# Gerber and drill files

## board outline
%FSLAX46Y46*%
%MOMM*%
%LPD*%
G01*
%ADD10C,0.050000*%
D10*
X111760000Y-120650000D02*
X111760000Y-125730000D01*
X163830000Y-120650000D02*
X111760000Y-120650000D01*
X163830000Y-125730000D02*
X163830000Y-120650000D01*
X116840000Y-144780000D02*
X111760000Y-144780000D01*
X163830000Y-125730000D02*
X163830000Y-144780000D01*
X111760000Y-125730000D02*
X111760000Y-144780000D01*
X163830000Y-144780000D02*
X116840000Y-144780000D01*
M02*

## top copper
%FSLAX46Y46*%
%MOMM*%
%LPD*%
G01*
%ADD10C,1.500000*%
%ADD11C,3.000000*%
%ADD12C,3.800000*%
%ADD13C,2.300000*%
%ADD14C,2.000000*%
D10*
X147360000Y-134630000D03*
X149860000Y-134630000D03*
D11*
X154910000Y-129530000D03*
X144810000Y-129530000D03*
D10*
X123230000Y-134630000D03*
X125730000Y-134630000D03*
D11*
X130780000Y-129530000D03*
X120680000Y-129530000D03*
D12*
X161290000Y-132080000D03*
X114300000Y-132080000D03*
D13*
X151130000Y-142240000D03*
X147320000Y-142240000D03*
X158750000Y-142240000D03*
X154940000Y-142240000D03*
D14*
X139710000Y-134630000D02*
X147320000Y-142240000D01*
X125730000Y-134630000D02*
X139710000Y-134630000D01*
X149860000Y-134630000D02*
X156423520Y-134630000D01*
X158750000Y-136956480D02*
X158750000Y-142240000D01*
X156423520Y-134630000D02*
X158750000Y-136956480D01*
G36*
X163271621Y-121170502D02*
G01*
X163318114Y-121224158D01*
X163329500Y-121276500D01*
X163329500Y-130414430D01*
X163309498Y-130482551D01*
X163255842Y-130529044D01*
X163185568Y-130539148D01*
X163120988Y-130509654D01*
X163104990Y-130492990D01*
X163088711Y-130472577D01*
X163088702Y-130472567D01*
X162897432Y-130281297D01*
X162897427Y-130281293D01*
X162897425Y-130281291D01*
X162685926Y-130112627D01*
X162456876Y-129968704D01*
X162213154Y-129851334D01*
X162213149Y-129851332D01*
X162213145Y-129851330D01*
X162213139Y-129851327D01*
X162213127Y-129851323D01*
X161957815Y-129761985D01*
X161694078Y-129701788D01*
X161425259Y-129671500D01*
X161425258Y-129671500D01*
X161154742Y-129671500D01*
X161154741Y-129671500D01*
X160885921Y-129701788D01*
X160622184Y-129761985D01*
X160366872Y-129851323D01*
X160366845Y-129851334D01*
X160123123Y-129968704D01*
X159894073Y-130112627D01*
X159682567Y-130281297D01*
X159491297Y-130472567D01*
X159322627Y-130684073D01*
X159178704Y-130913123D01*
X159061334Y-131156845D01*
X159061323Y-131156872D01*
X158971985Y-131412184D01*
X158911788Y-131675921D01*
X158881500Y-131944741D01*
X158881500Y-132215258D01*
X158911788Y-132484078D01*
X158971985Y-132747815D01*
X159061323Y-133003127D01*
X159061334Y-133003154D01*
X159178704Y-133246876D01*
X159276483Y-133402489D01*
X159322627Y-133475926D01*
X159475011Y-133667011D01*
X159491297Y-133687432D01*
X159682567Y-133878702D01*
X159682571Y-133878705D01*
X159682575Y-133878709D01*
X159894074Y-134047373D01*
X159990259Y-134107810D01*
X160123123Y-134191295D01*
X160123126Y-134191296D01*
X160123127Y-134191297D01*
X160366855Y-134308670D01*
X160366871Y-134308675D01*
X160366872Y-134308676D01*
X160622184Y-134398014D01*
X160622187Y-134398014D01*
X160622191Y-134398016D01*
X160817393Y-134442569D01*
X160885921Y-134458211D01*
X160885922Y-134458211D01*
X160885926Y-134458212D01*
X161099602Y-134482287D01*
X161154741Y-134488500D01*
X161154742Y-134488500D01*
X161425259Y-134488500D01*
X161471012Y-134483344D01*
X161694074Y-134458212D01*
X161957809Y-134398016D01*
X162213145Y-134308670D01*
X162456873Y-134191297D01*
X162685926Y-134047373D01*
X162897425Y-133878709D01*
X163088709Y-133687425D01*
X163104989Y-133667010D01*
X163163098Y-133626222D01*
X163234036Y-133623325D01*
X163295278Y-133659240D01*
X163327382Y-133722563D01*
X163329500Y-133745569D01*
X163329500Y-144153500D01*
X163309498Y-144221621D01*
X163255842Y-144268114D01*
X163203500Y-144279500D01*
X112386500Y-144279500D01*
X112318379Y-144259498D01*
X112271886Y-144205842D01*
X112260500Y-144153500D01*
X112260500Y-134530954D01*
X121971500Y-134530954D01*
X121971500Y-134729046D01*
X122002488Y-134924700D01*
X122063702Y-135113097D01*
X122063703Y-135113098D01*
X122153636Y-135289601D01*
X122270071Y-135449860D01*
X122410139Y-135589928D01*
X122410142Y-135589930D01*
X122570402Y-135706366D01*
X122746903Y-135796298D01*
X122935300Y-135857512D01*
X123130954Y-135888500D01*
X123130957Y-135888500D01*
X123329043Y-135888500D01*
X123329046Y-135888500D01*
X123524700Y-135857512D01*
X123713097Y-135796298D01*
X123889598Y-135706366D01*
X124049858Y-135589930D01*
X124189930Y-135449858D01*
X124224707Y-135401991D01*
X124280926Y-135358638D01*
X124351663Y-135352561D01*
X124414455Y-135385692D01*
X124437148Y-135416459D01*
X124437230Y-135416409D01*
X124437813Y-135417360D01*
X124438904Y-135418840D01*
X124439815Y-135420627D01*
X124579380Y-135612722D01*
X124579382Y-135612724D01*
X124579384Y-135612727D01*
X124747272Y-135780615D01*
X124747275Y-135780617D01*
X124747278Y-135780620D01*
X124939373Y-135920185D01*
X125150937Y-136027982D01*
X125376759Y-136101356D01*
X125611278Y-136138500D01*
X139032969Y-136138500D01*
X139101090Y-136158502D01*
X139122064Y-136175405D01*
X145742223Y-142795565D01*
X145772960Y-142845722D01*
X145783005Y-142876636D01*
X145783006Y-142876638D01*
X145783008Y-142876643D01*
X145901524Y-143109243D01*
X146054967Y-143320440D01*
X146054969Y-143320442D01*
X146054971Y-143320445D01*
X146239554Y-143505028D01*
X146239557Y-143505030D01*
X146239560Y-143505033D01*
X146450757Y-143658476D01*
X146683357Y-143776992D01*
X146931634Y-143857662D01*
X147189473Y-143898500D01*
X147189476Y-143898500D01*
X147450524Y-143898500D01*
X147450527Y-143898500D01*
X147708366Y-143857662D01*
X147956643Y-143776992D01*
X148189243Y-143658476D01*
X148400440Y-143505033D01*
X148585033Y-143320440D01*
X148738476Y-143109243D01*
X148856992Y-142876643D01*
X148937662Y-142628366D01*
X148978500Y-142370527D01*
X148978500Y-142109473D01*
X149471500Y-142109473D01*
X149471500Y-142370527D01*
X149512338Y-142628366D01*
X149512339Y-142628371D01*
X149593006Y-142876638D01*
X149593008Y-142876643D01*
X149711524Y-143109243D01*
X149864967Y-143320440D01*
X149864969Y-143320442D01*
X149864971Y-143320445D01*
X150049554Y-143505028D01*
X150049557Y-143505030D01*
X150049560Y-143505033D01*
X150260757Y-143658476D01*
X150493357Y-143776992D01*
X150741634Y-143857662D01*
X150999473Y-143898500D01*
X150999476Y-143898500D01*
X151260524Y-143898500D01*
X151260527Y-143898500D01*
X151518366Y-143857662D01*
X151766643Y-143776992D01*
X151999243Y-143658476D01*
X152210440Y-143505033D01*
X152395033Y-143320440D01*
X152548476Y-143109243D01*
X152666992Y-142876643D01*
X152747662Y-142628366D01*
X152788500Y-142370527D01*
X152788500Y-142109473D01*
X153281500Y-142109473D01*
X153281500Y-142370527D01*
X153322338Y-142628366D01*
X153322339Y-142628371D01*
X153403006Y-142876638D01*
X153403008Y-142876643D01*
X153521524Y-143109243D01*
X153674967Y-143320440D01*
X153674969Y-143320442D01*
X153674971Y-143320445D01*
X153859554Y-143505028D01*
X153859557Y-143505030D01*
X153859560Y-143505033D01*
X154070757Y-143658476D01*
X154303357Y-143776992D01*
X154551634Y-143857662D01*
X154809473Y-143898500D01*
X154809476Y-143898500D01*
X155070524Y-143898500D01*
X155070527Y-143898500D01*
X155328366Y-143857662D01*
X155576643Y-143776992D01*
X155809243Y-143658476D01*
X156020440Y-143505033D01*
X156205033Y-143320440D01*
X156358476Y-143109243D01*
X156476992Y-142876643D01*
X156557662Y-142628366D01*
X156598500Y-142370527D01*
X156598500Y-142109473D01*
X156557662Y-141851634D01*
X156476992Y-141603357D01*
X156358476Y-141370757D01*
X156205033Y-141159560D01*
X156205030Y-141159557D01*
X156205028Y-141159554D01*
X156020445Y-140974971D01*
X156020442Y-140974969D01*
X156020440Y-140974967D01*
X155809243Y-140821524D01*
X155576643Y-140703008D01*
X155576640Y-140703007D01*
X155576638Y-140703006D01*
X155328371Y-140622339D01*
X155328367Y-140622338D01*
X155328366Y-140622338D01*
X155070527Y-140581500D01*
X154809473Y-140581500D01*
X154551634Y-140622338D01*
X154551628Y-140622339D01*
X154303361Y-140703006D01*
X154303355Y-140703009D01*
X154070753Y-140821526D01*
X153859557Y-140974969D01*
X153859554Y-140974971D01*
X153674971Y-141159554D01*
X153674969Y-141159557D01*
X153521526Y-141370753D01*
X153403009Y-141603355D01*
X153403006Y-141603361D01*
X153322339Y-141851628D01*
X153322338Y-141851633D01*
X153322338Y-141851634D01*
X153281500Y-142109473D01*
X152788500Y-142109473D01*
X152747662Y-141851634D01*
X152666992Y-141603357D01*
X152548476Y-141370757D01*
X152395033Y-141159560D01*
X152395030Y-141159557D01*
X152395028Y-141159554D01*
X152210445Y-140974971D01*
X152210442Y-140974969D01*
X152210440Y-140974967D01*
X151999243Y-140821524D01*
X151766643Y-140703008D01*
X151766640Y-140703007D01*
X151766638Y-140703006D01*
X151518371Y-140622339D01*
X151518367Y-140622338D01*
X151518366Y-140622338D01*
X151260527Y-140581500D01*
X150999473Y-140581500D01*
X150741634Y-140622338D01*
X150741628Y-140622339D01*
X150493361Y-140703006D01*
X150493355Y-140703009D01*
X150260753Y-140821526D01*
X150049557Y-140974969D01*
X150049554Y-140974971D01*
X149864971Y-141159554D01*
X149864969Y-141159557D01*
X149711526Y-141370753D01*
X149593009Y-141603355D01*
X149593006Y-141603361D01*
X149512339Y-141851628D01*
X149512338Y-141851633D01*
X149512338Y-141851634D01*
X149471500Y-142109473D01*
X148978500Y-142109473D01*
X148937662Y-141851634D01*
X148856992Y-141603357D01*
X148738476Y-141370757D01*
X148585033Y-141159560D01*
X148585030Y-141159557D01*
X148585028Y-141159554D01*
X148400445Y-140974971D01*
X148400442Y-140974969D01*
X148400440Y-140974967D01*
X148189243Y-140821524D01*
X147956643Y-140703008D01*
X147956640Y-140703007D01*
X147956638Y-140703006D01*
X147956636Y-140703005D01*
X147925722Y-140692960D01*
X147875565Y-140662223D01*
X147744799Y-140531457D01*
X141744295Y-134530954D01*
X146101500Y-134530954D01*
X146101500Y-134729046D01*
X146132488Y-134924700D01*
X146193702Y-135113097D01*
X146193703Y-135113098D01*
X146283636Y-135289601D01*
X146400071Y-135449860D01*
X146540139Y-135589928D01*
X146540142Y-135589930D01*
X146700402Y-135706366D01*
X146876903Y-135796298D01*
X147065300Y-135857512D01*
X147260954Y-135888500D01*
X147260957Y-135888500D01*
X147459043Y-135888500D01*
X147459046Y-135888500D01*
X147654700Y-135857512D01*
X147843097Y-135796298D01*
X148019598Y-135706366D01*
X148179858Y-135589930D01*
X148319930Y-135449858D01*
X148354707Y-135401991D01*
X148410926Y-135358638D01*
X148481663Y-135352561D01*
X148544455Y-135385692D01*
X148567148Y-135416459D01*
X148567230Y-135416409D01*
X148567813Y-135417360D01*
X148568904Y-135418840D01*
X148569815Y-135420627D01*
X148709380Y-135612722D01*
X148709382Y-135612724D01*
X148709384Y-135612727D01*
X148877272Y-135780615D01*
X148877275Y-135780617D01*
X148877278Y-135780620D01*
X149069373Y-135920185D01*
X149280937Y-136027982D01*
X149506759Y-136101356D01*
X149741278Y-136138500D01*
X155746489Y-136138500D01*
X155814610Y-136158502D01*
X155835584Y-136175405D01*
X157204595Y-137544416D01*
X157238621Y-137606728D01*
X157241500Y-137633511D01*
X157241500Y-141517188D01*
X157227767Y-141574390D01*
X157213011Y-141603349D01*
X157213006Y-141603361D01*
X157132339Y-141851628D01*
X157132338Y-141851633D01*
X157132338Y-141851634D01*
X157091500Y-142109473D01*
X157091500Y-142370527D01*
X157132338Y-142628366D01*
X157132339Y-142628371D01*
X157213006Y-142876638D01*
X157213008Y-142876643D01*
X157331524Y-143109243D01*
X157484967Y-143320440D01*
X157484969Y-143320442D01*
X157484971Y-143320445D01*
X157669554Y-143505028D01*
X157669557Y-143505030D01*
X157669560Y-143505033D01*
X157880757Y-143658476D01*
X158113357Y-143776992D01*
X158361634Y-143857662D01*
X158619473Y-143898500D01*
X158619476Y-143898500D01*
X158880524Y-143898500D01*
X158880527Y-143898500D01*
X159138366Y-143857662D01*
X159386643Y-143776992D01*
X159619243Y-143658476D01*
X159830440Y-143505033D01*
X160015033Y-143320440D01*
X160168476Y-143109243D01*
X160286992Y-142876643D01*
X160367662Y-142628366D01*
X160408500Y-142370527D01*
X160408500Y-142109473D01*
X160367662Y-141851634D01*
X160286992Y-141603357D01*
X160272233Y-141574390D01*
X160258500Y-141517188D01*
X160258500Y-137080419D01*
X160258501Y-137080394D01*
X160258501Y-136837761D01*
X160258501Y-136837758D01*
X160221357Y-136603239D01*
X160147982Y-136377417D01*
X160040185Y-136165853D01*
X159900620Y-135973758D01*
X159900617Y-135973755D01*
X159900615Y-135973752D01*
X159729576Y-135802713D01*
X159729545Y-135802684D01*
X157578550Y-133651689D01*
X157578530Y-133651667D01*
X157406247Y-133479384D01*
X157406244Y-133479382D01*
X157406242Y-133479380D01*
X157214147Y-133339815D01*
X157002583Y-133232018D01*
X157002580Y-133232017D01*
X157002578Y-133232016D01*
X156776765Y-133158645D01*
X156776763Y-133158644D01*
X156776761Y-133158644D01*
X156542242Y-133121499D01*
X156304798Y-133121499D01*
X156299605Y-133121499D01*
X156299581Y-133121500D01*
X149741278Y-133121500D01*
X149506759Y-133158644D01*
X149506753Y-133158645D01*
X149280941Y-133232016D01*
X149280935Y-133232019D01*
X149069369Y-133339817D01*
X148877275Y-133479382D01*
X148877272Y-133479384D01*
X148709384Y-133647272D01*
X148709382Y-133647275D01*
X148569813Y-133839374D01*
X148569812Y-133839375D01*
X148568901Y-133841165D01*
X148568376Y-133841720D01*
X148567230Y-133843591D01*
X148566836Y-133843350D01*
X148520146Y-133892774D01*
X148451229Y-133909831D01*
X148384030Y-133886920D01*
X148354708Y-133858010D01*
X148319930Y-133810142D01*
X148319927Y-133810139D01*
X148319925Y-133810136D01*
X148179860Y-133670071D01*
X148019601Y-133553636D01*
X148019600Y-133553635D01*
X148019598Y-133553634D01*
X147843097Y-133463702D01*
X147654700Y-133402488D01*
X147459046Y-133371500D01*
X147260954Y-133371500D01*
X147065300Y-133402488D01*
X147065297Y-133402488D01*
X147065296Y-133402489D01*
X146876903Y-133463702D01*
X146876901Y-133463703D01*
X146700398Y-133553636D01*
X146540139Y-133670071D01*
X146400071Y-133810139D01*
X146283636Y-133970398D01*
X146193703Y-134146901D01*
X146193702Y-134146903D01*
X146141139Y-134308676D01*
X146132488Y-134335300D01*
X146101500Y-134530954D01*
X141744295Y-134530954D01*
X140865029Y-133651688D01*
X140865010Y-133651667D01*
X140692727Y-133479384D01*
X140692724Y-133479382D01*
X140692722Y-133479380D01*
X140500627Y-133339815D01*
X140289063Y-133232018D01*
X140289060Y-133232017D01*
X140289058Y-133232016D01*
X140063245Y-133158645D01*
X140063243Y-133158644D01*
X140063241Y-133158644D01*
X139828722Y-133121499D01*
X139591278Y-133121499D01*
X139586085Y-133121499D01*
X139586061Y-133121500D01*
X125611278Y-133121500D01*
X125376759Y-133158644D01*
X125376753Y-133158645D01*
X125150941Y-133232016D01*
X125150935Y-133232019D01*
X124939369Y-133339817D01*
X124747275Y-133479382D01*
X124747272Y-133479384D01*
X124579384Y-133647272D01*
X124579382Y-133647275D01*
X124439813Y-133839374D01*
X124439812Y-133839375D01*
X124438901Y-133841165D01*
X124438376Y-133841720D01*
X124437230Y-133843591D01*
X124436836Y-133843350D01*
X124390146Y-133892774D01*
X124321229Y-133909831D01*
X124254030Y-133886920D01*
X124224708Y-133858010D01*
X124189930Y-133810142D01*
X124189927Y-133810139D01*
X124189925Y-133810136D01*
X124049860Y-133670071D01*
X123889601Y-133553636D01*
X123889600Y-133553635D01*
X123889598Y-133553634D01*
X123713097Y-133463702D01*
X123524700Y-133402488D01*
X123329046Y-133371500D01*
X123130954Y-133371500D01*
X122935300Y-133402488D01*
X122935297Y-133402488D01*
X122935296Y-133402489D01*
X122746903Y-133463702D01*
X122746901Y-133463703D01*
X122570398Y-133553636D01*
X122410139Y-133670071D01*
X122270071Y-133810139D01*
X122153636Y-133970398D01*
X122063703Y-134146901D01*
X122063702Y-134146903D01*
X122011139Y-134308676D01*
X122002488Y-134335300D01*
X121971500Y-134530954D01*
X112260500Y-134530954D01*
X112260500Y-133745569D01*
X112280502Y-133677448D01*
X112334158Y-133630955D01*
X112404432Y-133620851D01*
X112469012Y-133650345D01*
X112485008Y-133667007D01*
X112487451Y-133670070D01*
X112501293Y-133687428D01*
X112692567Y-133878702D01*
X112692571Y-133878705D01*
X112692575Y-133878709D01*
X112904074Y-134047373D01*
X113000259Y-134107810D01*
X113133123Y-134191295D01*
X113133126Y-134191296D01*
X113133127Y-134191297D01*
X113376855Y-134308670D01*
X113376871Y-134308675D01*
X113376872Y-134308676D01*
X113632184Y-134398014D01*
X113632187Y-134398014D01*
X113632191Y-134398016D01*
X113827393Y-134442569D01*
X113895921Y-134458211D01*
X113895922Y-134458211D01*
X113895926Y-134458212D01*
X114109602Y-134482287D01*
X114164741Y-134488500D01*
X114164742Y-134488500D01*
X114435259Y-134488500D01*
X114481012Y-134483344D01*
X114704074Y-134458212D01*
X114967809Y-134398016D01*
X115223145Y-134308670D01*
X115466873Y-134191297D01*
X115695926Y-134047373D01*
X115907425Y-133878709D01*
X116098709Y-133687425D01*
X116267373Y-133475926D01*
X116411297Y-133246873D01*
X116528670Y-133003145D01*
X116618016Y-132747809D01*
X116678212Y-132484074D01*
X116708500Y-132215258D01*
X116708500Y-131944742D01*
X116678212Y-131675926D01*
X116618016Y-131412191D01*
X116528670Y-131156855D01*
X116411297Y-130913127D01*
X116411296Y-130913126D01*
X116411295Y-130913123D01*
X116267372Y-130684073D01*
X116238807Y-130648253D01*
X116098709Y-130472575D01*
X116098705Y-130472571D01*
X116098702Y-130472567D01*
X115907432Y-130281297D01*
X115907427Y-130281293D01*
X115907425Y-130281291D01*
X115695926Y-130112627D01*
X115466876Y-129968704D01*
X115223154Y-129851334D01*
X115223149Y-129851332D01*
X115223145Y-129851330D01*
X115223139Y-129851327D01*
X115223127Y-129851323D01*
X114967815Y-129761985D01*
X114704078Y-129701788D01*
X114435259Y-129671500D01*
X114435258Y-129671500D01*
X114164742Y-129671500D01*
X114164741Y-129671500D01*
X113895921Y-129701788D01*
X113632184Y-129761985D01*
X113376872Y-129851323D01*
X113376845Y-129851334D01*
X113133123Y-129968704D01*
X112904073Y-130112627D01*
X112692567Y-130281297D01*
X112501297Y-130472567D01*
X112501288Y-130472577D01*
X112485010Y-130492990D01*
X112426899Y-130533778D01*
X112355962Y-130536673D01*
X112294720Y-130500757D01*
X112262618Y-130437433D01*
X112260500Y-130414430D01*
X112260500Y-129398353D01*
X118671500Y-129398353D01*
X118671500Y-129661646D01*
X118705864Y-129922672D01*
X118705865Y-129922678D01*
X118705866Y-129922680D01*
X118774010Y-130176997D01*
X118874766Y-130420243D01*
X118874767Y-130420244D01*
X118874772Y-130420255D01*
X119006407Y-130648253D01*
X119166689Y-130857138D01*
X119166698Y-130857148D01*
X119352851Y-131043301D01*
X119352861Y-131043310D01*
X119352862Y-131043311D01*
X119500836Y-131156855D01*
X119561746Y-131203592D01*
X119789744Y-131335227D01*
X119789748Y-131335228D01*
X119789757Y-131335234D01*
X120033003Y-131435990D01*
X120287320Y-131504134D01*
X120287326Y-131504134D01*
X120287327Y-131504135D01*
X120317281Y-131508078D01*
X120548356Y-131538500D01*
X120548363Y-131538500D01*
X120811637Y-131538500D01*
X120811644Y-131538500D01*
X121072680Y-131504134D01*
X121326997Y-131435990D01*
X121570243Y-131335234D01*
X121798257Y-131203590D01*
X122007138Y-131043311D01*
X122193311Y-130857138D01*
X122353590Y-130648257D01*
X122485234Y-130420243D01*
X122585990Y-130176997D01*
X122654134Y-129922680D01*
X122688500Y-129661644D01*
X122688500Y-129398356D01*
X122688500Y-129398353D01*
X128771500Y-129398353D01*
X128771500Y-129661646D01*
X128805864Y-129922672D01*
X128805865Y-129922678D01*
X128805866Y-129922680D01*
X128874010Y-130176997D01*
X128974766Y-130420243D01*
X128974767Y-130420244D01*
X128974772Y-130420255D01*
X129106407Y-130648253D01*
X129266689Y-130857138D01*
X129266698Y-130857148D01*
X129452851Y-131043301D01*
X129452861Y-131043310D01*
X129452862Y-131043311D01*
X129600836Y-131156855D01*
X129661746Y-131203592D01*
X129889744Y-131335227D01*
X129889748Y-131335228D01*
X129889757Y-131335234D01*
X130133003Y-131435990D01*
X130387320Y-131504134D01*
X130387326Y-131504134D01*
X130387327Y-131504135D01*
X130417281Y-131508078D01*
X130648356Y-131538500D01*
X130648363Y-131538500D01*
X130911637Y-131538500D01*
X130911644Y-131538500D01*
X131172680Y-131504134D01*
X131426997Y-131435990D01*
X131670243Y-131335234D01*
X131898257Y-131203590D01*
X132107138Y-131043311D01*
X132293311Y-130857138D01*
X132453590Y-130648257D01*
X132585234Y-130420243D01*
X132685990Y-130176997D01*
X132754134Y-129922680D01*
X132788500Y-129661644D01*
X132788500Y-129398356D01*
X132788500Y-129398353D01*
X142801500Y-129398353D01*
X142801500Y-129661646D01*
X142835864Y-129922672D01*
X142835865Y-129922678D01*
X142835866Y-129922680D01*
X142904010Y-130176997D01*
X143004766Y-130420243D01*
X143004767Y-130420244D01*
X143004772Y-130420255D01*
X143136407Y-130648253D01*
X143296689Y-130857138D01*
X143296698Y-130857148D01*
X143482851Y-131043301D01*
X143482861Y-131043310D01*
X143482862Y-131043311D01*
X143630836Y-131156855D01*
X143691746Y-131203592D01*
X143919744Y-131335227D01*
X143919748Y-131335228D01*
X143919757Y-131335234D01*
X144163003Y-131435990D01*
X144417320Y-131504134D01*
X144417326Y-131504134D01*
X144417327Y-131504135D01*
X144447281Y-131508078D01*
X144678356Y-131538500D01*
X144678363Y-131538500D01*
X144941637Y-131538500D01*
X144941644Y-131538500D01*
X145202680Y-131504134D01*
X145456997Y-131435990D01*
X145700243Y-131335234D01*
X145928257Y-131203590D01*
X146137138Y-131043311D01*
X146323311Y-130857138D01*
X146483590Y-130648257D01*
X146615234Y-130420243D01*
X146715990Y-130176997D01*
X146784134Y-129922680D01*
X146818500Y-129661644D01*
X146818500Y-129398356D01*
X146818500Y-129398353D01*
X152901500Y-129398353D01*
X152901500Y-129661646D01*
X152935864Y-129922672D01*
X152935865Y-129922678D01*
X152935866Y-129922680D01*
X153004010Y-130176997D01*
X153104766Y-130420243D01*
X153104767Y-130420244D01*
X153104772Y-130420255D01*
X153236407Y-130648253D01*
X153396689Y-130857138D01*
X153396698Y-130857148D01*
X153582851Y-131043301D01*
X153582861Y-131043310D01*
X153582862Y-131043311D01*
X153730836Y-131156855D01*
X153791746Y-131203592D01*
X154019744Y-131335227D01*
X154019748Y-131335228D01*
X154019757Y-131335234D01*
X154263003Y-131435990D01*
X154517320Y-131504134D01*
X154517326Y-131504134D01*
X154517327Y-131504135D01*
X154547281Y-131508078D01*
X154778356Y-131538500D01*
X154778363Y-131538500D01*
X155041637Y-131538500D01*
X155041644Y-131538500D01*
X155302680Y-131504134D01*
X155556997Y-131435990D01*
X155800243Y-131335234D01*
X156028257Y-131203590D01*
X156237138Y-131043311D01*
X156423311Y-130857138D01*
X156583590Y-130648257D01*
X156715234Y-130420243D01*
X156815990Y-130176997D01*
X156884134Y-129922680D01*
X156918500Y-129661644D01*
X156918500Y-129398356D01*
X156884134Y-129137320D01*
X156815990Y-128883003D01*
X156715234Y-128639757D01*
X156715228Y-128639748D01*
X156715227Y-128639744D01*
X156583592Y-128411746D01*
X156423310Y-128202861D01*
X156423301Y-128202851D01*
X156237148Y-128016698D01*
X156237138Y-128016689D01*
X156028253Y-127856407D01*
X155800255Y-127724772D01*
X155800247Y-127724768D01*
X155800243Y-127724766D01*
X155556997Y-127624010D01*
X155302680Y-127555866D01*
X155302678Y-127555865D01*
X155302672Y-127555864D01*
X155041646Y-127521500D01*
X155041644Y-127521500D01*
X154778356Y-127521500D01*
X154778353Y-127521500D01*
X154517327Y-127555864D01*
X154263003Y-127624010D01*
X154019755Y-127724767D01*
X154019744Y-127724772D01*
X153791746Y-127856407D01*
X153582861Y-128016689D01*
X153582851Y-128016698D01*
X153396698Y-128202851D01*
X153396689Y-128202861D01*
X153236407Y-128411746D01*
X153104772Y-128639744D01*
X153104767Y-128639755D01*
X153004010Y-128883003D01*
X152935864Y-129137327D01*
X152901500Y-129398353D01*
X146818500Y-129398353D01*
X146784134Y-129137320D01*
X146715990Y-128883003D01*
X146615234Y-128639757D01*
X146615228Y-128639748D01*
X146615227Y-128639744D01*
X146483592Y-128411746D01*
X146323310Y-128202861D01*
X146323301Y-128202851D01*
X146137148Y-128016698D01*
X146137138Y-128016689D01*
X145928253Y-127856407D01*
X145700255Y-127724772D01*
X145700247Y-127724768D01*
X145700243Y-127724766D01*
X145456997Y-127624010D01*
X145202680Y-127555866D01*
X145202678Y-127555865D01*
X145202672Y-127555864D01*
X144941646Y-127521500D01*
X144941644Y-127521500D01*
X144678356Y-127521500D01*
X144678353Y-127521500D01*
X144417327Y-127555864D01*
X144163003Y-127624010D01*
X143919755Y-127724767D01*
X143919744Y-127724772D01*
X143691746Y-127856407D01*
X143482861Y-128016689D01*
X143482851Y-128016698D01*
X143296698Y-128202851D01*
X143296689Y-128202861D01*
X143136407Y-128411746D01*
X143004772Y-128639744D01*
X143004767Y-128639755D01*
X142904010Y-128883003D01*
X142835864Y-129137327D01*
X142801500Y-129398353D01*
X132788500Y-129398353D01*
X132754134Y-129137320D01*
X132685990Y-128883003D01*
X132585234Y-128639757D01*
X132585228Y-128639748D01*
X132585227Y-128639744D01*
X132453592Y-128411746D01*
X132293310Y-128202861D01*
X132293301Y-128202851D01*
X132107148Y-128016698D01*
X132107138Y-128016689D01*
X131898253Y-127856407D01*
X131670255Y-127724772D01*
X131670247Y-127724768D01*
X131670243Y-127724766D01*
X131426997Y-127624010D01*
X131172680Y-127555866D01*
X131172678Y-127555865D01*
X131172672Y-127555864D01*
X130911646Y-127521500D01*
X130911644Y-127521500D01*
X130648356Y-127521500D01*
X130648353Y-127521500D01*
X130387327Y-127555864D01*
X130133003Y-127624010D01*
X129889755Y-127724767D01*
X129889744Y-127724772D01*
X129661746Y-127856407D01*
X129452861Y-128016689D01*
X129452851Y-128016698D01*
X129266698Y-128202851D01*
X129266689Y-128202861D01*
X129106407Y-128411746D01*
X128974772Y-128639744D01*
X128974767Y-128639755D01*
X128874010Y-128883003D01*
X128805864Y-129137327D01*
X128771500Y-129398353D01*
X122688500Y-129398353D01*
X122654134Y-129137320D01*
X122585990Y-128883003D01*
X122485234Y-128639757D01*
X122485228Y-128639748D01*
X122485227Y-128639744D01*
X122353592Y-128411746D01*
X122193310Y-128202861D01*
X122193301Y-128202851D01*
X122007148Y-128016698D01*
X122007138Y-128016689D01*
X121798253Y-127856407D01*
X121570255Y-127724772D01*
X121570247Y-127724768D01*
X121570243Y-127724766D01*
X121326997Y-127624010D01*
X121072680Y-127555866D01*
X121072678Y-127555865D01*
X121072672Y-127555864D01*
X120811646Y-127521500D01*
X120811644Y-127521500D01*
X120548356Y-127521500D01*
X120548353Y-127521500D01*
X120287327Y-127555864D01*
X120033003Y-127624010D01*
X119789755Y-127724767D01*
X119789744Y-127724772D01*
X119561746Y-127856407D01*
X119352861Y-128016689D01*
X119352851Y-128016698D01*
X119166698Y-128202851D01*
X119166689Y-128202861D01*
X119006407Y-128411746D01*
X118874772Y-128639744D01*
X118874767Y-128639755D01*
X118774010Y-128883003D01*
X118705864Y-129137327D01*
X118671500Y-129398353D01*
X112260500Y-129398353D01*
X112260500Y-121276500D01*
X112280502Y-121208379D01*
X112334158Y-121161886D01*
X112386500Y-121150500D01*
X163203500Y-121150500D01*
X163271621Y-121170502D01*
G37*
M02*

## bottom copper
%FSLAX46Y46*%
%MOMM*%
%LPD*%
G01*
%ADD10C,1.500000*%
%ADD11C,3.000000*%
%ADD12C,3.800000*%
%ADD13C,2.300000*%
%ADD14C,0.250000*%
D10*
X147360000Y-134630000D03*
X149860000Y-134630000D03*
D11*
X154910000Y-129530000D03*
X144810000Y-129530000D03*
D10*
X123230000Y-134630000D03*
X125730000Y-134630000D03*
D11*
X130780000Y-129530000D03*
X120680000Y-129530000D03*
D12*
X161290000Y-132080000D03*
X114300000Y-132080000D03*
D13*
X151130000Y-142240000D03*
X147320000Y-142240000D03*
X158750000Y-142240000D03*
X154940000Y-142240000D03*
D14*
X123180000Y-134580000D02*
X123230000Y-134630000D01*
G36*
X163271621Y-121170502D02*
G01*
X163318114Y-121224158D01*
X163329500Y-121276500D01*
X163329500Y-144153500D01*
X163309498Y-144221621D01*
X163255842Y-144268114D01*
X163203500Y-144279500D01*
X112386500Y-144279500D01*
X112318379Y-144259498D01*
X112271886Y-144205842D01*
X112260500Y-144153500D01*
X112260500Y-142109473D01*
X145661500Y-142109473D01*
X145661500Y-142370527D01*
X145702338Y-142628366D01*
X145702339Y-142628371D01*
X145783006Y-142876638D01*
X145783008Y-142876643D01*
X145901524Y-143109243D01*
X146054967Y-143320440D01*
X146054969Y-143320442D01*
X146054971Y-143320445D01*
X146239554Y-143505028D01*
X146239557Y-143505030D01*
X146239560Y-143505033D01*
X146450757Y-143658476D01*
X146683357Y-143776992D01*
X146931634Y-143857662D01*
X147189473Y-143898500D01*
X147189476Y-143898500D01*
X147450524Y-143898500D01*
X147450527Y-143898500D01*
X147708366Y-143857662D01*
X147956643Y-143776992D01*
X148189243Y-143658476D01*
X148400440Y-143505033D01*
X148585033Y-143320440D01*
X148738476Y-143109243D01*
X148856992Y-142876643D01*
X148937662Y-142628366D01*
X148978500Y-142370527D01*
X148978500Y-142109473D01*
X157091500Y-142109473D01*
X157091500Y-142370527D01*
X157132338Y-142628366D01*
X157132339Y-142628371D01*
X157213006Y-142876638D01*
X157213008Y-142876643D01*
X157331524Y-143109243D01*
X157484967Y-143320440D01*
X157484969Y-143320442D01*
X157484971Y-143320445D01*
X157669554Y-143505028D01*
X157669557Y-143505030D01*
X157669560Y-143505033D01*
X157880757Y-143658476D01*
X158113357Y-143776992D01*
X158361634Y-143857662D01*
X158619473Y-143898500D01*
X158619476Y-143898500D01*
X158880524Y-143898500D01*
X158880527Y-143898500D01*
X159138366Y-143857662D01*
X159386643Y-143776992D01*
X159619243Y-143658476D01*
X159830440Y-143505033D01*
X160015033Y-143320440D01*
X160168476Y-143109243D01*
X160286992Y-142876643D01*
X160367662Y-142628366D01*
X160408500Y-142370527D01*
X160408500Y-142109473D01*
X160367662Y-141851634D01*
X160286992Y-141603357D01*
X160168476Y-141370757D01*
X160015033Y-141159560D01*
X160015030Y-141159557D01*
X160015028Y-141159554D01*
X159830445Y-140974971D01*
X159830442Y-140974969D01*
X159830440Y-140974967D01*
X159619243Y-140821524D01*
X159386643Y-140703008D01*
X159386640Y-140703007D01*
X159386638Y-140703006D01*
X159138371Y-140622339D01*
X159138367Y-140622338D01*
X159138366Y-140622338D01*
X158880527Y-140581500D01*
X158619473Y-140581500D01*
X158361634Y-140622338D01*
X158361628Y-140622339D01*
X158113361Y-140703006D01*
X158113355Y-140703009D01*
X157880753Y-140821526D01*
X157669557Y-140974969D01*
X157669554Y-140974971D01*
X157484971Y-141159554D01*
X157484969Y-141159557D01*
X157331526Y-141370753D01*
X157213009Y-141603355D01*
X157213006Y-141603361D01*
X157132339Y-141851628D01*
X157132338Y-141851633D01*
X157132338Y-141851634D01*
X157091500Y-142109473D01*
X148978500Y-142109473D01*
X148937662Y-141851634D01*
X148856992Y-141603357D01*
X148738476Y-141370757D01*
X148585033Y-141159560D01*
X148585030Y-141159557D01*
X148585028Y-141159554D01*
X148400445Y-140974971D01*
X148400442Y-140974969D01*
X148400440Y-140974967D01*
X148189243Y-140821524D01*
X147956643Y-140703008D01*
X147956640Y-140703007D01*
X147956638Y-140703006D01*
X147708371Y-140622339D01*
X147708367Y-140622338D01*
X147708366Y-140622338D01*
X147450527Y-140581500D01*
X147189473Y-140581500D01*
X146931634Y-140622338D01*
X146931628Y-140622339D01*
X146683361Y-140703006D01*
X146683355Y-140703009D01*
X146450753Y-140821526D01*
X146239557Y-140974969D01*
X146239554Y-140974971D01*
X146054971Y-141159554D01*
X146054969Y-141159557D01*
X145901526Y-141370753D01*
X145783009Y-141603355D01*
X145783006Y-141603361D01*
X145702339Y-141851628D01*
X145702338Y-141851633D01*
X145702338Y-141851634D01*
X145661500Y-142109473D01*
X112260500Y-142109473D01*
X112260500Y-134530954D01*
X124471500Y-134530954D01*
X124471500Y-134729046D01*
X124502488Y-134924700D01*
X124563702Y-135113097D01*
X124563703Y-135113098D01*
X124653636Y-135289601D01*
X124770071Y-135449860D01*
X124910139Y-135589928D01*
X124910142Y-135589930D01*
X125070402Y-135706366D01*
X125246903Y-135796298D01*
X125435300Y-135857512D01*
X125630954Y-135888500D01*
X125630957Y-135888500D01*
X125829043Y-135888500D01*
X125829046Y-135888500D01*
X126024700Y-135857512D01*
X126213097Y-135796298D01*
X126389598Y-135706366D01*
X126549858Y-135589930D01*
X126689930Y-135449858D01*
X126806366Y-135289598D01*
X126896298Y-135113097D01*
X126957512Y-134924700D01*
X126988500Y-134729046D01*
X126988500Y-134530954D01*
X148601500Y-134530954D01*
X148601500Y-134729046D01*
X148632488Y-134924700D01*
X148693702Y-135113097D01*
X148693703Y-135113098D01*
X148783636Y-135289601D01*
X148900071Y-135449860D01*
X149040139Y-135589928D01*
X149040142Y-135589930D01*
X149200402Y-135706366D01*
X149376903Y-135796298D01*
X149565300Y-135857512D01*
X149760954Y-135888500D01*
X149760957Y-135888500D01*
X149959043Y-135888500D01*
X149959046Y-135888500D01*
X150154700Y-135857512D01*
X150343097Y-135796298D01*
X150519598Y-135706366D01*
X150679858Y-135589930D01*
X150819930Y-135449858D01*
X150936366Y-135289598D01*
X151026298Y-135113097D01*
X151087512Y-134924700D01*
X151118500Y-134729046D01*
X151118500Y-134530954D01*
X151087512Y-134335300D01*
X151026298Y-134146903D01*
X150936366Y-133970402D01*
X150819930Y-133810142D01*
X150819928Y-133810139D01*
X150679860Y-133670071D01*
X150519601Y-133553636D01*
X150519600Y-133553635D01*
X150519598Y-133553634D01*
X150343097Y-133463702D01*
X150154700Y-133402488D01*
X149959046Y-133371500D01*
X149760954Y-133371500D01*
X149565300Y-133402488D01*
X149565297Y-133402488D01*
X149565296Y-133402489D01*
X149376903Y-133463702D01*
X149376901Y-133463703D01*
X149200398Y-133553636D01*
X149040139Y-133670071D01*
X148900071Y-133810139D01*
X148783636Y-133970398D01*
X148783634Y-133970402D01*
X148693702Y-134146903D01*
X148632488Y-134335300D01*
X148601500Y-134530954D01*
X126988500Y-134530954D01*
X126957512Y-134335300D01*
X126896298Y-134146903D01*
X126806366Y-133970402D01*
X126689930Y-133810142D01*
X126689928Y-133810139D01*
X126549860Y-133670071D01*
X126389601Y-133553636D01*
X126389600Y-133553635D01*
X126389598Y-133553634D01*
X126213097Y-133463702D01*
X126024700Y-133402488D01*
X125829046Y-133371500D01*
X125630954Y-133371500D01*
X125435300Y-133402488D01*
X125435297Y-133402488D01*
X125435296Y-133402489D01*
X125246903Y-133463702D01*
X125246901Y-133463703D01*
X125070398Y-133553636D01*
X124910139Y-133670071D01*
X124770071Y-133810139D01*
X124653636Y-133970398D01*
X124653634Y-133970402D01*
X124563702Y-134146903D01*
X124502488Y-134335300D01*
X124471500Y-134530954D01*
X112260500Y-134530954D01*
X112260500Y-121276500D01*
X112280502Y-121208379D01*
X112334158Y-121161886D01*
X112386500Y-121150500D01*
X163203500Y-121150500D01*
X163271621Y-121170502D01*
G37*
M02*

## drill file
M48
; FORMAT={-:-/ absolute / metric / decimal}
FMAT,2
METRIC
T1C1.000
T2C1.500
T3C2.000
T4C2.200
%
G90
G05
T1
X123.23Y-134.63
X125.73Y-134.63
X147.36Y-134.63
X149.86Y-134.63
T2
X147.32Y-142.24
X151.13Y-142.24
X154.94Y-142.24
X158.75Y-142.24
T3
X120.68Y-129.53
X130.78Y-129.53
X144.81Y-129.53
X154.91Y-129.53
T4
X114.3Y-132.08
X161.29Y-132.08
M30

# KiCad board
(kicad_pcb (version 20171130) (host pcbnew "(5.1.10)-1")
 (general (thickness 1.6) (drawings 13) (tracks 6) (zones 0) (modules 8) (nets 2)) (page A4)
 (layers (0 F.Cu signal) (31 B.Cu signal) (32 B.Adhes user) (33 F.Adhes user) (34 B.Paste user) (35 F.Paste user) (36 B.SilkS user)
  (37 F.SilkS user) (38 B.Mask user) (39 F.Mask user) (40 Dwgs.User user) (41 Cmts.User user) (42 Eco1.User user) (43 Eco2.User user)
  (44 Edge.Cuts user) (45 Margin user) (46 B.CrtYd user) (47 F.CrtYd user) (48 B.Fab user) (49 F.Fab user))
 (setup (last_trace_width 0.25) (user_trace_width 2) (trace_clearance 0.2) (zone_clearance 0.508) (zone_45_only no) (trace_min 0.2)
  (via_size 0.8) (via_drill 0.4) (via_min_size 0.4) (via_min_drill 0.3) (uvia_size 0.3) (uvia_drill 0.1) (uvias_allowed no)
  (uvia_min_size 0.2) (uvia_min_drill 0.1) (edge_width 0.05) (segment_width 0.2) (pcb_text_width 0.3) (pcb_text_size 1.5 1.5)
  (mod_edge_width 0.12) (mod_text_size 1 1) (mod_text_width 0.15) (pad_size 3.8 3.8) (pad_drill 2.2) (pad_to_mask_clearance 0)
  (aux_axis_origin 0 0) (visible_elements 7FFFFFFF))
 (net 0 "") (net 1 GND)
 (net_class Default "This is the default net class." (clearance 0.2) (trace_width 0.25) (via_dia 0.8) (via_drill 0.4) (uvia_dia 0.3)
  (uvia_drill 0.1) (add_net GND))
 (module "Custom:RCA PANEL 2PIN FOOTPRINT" (layer F.Cu) (at 149.86 132.08 270)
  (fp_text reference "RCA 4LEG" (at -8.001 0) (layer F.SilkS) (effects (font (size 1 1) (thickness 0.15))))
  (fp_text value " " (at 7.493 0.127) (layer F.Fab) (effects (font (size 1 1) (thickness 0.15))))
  (pad 4 thru_hole circle (at 2.55 2.5 270) (size 1.5 1.5) (drill 1) (layers *.Cu *.Mask) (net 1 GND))
  (pad 3 thru_hole circle (at 2.55 0 270) (size 1.5 1.5) (drill 1) (layers *.Cu *.Mask))
  (pad 2 thru_hole circle (at -2.55 -5.05 270) (size 3 3) (drill 2) (layers *.Cu *.Mask) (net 1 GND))
  (pad 1 thru_hole circle (at -2.55 5.05 270) (size 3 3) (drill 2) (layers *.Cu *.Mask) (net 1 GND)))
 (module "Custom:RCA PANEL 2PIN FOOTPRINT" (layer F.Cu) (at 125.73 132.08 270)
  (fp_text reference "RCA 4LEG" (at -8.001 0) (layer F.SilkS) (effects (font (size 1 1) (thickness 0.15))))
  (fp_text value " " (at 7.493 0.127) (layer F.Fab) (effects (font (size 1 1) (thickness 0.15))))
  (pad 4 thru_hole circle (at 2.55 2.5 270) (size 1.5 1.5) (drill 1) (layers *.Cu *.Mask) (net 1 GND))
  (pad 3 thru_hole circle (at 2.55 0 270) (size 1.5 1.5) (drill 1) (layers *.Cu *.Mask))
  (pad 2 thru_hole circle (at -2.55 -5.05 270) (size 3 3) (drill 2) (layers *.Cu *.Mask) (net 1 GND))
  (pad 1 thru_hole circle (at -2.55 5.05 270) (size 3 3) (drill 2) (layers *.Cu *.Mask) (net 1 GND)))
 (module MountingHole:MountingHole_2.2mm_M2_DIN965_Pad (layer F.Cu) (at 161.29 132.08)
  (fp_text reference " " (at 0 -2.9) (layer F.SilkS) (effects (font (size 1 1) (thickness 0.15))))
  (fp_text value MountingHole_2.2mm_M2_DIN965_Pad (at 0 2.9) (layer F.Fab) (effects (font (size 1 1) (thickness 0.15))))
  (pad 1 thru_hole circle (at 0 0) (size 3.8 3.8) (drill 2.2) (layers *.Cu *.Mask) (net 1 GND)))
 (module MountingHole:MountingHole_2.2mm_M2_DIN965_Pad (layer F.Cu) (at 114.3 132.08)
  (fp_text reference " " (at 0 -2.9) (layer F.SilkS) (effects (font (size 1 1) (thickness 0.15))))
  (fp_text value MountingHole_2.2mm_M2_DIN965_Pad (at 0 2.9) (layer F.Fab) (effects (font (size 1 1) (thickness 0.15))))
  (pad 1 thru_hole circle (at 0 0) (size 3.8 3.8) (drill 2.2) (layers *.Cu *.Mask) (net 1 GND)))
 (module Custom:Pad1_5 (layer F.Cu) (at 151.13 142.24)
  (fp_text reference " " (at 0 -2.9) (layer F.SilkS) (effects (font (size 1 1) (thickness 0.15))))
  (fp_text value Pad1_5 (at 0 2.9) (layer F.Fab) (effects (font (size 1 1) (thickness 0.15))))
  (pad 1 thru_hole circle (at 0 0) (size 2.3 2.3) (drill 1.5) (layers *.Cu *.Mask) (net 1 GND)))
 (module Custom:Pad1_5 (layer F.Cu) (at 147.32 142.24)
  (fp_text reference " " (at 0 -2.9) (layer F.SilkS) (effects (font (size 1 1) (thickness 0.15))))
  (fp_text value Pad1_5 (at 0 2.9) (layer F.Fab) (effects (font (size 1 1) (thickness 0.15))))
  (pad 1 thru_hole circle (at 0 0) (size 2.3 2.3) (drill 1.5) (layers *.Cu *.Mask)))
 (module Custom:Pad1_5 (layer F.Cu) (at 158.75 142.24)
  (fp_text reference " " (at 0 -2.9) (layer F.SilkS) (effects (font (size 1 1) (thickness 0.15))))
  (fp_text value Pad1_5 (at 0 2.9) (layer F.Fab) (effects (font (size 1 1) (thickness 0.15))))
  (pad 1 thru_hole circle (at 0 0) (size 2.3 2.3) (drill 1.5) (layers *.Cu *.Mask)))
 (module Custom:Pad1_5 (layer F.Cu) (at 154.94 142.24)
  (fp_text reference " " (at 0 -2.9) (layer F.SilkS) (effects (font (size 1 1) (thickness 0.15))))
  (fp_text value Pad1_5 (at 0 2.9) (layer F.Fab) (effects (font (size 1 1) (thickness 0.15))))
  (pad 1 thru_hole circle (at 0 0) (size 2.3 2.3) (drill 1.5) (layers *.Cu *.Mask) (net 1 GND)))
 (gr_line (start 111.76 120.65) (end 111.76 125.73) (layer Edge.Cuts) (width 0.05))
 (gr_line (start 163.83 120.65) (end 111.76 120.65) (layer Edge.Cuts) (width 0.05))
 (gr_line (start 163.83 125.73) (end 163.83 120.65) (layer Edge.Cuts) (width 0.05))
 (gr_line (start 116.84 144.78) (end 111.76 144.78) (layer Edge.Cuts) (width 0.05))
 (gr_line (start 163.83 125.73) (end 163.83 144.78) (layer Edge.Cuts) (width 0.05))
 (gr_line (start 111.76 125.73) (end 111.76 144.78) (layer Edge.Cuts) (width 0.05))
 (gr_line (start 163.83 144.78) (end 116.84 144.78) (layer Edge.Cuts) (width 0.05))
 (segment (start 139.71 134.63) (end 147.32 142.24) (width 2) (layer F.Cu) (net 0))
 (segment (start 125.73 134.63) (end 139.71 134.63) (width 2) (layer F.Cu) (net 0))
 (segment (start 149.86 134.63) (end 156.42352 134.63) (width 2) (layer F.Cu) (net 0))
 (segment (start 158.75 136.95648) (end 158.75 142.24) (width 2) (layer F.Cu) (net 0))
 (segment (start 156.42352 134.63) (end 158.75 136.95648) (width 2) (layer F.Cu) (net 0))
 (segment (start 123.18 134.58) (end 123.23 134.63) (width 0.25) (layer B.Cu) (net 1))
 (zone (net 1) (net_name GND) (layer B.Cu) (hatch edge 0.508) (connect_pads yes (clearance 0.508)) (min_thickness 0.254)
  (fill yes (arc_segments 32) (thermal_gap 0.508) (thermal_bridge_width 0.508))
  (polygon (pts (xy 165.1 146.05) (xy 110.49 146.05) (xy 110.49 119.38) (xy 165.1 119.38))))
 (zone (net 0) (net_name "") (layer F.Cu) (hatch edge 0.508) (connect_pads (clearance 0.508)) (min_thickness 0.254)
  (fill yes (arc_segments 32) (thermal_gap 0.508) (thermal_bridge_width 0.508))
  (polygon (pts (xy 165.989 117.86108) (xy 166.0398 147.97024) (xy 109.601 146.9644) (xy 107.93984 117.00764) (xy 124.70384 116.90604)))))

